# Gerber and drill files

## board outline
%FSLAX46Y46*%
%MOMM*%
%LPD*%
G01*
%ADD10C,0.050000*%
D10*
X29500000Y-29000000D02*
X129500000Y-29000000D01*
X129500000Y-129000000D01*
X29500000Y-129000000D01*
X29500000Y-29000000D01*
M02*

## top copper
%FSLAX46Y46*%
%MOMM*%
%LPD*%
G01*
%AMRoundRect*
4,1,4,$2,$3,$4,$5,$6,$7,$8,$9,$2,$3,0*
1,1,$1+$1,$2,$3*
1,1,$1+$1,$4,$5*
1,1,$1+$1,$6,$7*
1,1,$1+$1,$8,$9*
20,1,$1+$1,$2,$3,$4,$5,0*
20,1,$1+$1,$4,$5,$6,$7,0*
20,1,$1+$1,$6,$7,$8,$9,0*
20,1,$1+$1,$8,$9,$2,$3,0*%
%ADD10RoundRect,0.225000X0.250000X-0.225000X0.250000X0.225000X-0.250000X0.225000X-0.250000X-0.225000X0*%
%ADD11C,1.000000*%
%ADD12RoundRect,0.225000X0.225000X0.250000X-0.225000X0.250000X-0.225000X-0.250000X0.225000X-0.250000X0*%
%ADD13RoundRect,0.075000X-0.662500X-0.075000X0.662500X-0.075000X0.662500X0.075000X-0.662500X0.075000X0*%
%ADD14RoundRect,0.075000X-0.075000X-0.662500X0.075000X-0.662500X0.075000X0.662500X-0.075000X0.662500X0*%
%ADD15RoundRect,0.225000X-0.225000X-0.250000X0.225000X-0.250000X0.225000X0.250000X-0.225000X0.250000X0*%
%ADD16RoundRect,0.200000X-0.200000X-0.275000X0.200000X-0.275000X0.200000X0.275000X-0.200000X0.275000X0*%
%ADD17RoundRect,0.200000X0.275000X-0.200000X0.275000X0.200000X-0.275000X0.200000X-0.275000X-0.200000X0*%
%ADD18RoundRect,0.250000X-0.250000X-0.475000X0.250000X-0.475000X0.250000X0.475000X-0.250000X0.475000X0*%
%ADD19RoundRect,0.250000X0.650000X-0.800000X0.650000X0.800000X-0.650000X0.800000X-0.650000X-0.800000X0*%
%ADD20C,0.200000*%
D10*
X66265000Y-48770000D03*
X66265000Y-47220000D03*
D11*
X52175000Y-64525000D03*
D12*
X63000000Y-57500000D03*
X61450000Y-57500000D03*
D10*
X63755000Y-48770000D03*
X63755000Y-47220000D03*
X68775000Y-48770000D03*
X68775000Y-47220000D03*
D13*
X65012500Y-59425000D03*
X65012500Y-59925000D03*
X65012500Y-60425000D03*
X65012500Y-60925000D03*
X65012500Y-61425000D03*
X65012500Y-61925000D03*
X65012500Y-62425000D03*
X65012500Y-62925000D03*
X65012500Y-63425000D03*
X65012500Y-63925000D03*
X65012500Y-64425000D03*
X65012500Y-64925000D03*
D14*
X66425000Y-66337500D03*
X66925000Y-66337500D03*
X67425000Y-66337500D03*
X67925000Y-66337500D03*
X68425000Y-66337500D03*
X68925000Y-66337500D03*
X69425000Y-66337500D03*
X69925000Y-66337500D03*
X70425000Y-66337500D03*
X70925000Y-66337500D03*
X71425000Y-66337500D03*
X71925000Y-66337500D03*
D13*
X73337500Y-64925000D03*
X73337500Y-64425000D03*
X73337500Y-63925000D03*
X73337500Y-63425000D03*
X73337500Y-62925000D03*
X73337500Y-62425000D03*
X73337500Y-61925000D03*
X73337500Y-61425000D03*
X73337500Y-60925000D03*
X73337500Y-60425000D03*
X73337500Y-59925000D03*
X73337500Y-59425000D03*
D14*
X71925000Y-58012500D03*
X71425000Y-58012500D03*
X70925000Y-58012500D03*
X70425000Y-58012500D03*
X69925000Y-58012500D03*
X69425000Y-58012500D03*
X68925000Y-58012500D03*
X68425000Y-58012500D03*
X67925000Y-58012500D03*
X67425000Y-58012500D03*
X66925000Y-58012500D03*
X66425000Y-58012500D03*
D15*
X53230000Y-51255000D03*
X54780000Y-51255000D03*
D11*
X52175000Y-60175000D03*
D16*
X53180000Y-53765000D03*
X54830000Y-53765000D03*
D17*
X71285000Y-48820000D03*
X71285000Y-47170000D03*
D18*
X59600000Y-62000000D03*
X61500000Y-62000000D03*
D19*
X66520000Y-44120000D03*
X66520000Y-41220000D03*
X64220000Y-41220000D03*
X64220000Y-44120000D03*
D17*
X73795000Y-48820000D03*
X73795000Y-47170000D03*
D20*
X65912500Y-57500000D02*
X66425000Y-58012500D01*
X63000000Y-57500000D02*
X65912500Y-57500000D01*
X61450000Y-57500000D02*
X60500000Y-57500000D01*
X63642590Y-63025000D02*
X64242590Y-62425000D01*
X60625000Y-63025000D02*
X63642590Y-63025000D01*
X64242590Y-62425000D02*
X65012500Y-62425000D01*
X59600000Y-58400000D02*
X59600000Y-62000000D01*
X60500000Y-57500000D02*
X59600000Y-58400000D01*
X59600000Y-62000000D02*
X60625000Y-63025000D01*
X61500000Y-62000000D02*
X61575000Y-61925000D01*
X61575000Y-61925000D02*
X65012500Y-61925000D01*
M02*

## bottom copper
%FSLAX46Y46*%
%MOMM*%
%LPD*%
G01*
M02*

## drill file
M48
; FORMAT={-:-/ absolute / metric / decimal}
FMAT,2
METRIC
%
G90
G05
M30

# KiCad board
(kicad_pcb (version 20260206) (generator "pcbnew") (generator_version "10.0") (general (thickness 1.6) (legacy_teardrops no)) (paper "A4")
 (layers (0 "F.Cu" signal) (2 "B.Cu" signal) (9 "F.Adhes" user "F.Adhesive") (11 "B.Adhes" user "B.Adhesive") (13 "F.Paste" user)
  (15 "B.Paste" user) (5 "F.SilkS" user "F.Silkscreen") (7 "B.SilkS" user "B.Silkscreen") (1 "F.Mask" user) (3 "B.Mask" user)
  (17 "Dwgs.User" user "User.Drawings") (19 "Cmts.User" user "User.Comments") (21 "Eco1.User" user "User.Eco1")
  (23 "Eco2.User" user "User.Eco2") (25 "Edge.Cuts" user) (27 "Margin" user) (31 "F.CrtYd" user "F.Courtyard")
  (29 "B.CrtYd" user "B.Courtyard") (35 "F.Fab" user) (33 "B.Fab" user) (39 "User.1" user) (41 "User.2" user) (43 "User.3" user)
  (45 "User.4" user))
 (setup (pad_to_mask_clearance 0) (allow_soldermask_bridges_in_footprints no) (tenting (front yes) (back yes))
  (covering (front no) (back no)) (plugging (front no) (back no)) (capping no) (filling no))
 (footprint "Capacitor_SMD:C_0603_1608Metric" (layer "F.Cu") (at 66.265 47.995 90)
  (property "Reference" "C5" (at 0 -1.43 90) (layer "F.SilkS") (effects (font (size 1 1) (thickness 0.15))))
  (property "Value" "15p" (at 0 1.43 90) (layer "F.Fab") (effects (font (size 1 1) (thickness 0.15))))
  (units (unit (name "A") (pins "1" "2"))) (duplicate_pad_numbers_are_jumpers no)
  (pad "1" smd roundrect (at -0.775 0 90) (size 0.9 0.95) (layers "F.Cu" "F.Mask" "F.Paste") (roundrect_rratio 0.25) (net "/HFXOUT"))
  (pad "2" smd roundrect (at 0.775 0 90) (size 0.9 0.95) (layers "F.Cu" "F.Mask" "F.Paste") (roundrect_rratio 0.25) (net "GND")))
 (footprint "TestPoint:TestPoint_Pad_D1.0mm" (layer "F.Cu") (at 52.175 64.525)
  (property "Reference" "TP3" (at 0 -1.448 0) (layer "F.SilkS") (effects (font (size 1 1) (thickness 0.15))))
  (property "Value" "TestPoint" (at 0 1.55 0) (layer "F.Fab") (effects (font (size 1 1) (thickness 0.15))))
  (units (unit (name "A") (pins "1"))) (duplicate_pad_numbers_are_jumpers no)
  (pad "1" smd circle (at 0 0) (size 1 1) (layers "F.Cu" "F.Mask") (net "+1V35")))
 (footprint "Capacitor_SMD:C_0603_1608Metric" (layer "F.Cu") (at 62.225 57.5 180)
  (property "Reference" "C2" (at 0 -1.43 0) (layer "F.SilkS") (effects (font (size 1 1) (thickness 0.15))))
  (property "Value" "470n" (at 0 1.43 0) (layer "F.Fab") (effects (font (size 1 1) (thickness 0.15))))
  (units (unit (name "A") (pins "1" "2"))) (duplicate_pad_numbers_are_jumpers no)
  (pad "1" smd roundrect (at -0.775 0 180) (size 0.9 0.95) (layers "F.Cu" "F.Mask" "F.Paste") (roundrect_rratio 0.25) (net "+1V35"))
  (pad "2" smd roundrect (at 0.775 0 180) (size 0.9 0.95) (layers "F.Cu" "F.Mask" "F.Paste") (roundrect_rratio 0.25) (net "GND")))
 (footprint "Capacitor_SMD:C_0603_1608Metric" (layer "F.Cu") (at 63.755 47.995 90)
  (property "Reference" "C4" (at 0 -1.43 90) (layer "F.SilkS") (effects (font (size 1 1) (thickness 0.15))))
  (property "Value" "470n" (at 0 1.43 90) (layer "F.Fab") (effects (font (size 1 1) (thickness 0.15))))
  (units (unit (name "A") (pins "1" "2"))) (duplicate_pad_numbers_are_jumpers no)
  (pad "1" smd roundrect (at -0.775 0 90) (size 0.9 0.95) (layers "F.Cu" "F.Mask" "F.Paste") (roundrect_rratio 0.25) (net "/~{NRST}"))
  (pad "2" smd roundrect (at 0.775 0 90) (size 0.9 0.95) (layers "F.Cu" "F.Mask" "F.Paste") (roundrect_rratio 0.25) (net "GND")))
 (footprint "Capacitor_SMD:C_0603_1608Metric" (layer "F.Cu") (at 68.775 47.995 90)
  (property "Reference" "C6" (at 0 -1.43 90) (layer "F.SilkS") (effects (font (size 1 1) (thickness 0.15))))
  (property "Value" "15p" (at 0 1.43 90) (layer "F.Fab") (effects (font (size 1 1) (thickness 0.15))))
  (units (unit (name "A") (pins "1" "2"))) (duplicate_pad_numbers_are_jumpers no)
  (pad "1" smd roundrect (at -0.775 0 90) (size 0.9 0.95) (layers "F.Cu" "F.Mask" "F.Paste") (roundrect_rratio 0.25) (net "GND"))
  (pad "2" smd roundrect (at 0.775 0 90) (size 0.9 0.95) (layers "F.Cu" "F.Mask" "F.Paste") (roundrect_rratio 0.25) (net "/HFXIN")))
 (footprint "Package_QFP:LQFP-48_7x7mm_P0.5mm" (layer "F.Cu") (at 69.175 62.175)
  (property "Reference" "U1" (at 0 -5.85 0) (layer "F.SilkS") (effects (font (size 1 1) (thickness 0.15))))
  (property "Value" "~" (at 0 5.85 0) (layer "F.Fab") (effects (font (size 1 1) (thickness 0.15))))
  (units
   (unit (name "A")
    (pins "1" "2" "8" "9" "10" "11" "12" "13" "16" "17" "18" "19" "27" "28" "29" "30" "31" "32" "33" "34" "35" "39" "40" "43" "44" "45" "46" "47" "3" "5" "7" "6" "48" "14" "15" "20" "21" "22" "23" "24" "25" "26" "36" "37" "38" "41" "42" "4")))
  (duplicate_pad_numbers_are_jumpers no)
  (pad "1" smd roundrect (at -4.1625 -2.75) (size 1.475 0.3) (layers "F.Cu" "F.Mask" "F.Paste") (roundrect_rratio 0.25)
   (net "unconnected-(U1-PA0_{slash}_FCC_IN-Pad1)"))
  (pad "2" smd roundrect (at -4.1625 -2.25) (size 1.475 0.3) (layers "F.Cu" "F.Mask" "F.Paste") (roundrect_rratio 0.25)
   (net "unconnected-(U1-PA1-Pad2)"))
  (pad "3" smd roundrect (at -4.1625 -1.75) (size 1.475 0.3) (layers "F.Cu" "F.Mask" "F.Paste") (roundrect_rratio 0.25)
   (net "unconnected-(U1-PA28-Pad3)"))
  (pad "4" smd roundrect (at -4.1625 -1.25) (size 1.475 0.3) (layers "F.Cu" "F.Mask" "F.Paste") (roundrect_rratio 0.25) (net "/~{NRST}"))
  (pad "5" smd roundrect (at -4.1625 -0.75) (size 1.475 0.3) (layers "F.Cu" "F.Mask" "F.Paste") (roundrect_rratio 0.25)
   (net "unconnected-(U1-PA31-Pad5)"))
  (pad "6" smd roundrect (at -4.1625 -0.25) (size 1.475 0.3) (layers "F.Cu" "F.Mask" "F.Paste") (roundrect_rratio 0.25) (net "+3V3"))
  (pad "7" smd roundrect (at -4.1625 0.25) (size 1.475 0.3) (layers "F.Cu" "F.Mask" "F.Paste") (roundrect_rratio 0.25) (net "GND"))
  (pad "8" smd roundrect (at -4.1625 0.75) (size 1.475 0.3) (layers "F.Cu" "F.Mask" "F.Paste") (roundrect_rratio 0.25) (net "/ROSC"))
  (pad "9" smd roundrect (at -4.1625 1.25) (size 1.475 0.3) (layers "F.Cu" "F.Mask" "F.Paste") (roundrect_rratio 0.25)
   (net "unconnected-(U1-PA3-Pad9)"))
  (pad "10" smd roundrect (at -4.1625 1.75) (size 1.475 0.3) (layers "F.Cu" "F.Mask" "F.Paste") (roundrect_rratio 0.25)
   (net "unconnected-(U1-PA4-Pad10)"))
  (pad "11" smd roundrect (at -4.1625 2.25) (size 1.475 0.3) (layers "F.Cu" "F.Mask" "F.Paste") (roundrect_rratio 0.25) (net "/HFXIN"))
  (pad "12" smd roundrect (at -4.1625 2.75) (size 1.475 0.3) (layers "F.Cu" "F.Mask" "F.Paste") (roundrect_rratio 0.25) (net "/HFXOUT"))
  (pad "13" smd roundrect (at -2.75 4.1625) (size 0.3 1.475) (layers "F.Cu" "F.Mask" "F.Paste") (roundrect_rratio 0.25)
   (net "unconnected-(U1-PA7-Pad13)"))
  (pad "14" smd roundrect (at -2.25 4.1625) (size 0.3 1.475) (layers "F.Cu" "F.Mask" "F.Paste") (roundrect_rratio 0.25)
   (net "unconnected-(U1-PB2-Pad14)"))
  (pad "15" smd roundrect (at -1.75 4.1625) (size 0.3 1.475) (layers "F.Cu" "F.Mask" "F.Paste") (roundrect_rratio 0.25)
   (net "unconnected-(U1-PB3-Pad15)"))
  (pad "16" smd roundrect (at -1.25 4.1625) (size 0.3 1.475) (layers "F.Cu" "F.Mask" "F.Paste") (roundrect_rratio 0.25)
   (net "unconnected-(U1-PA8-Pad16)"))
  (pad "17" smd roundrect (at -0.75 4.1625) (size 0.3 1.475) (layers "F.Cu" "F.Mask" "F.Paste") (roundrect_rratio 0.25)
   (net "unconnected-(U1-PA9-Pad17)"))
  (pad "18" smd roundrect (at -0.25 4.1625) (size 0.3 1.475) (layers "F.Cu" "F.Mask" "F.Paste") (roundrect_rratio 0.25)
   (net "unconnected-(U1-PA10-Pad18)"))
  (pad "19" smd roundrect (at 0.25 4.1625) (size 0.3 1.475) (layers "F.Cu" "F.Mask" "F.Paste") (roundrect_rratio 0.25)
   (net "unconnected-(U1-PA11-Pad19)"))
  (pad "20" smd roundrect (at 0.75 4.1625) (size 0.3 1.475) (layers "F.Cu" "F.Mask" "F.Paste") (roundrect_rratio 0.25)
   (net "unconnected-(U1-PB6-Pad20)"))
  (pad "21" smd roundrect (at 1.25 4.1625) (size 0.3 1.475) (layers "F.Cu" "F.Mask" "F.Paste") (roundrect_rratio 0.25)
   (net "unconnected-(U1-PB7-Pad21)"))
  (pad "22" smd roundrect (at 1.75 4.1625) (size 0.3 1.475) (layers "F.Cu" "F.Mask" "F.Paste") (roundrect_rratio 0.25)
   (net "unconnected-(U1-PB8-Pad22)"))
  (pad "23" smd roundrect (at 2.25 4.1625) (size 0.3 1.475) (layers "F.Cu" "F.Mask" "F.Paste") (roundrect_rratio 0.25)
   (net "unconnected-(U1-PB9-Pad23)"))
  (pad "24" smd roundrect (at 2.75 4.1625) (size 0.3 1.475) (layers "F.Cu" "F.Mask" "F.Paste") (roundrect_rratio 0.25)
   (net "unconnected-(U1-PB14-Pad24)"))
  (pad "25" smd roundrect (at 4.1625 2.75) (size 1.475 0.3) (layers "F.Cu" "F.Mask" "F.Paste") (roundrect_rratio 0.25)
   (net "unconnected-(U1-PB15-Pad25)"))
  (pad "26" smd roundrect (at 4.1625 2.25) (size 1.475 0.3) (layers "F.Cu" "F.Mask" "F.Paste") (roundrect_rratio 0.25)
   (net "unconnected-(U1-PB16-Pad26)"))
  (pad "27" smd roundrect (at 4.1625 1.75) (size 1.475 0.3) (layers "F.Cu" "F.Mask" "F.Paste") (roundrect_rratio 0.25)
   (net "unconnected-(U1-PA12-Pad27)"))
  (pad "28" smd roundrect (at 4.1625 1.25) (size 1.475 0.3) (layers "F.Cu" "F.Mask" "F.Paste") (roundrect_rratio 0.25)
   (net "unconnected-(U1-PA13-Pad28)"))
  (pad "29" smd roundrect (at 4.1625 0.75) (size 1.475 0.3) (layers "F.Cu" "F.Mask" "F.Paste") (roundrect_rratio 0.25)
   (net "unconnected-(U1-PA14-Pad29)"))
  (pad "30" smd roundrect (at 4.1625 0.25) (size 1.475 0.3) (layers "F.Cu" "F.Mask" "F.Paste") (roundrect_rratio 0.25)
   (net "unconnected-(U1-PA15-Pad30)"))
  (pad "31" smd roundrect (at 4.1625 -0.25) (size 1.475 0.3) (layers "F.Cu" "F.Mask" "F.Paste") (roundrect_rratio 0.25)
   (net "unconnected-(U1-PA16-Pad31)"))
  (pad "32" smd roundrect (at 4.1625 -0.75) (size 1.475 0.3) (layers "F.Cu" "F.Mask" "F.Paste") (roundrect_rratio 0.25)
   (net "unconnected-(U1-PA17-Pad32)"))
  (pad "33" smd roundrect (at 4.1625 -1.25) (size 1.475 0.3) (layers "F.Cu" "F.Mask" "F.Paste") (roundrect_rratio 0.25)
   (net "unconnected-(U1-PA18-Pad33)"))
  (pad "34" smd roundrect (at 4.1625 -1.75) (size 1.475 0.3) (layers "F.Cu" "F.Mask" "F.Paste") (roundrect_rratio 0.25)
   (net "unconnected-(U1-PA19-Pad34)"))
  (pad "35" smd roundrect (at 4.1625 -2.25) (size 1.475 0.3) (layers "F.Cu" "F.Mask" "F.Paste") (roundrect_rratio 0.25)
   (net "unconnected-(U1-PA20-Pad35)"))
  (pad "36" smd roundrect (at 4.1625 -2.75) (size 1.475 0.3) (layers "F.Cu" "F.Mask" "F.Paste") (roundrect_rratio 0.25)
   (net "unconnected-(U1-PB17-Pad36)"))
  (pad "37" smd roundrect (at 2.75 -4.1625) (size 0.3 1.475) (layers "F.Cu" "F.Mask" "F.Paste") (roundrect_rratio 0.25)
   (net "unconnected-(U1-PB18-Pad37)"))
  (pad "38" smd roundrect (at 2.25 -4.1625) (size 0.3 1.475) (layers "F.Cu" "F.Mask" "F.Paste") (roundrect_rratio 0.25)
   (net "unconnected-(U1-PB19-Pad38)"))
  (pad "39" smd roundrect (at 1.75 -4.1625) (size 0.3 1.475) (layers "F.Cu" "F.Mask" "F.Paste") (roundrect_rratio 0.25) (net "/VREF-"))
  (pad "40" smd roundrect (at 1.25 -4.1625) (size 0.3 1.475) (layers "F.Cu" "F.Mask" "F.Paste") (roundrect_rratio 0.25)
   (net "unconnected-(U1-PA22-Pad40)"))
  (pad "41" smd roundrect (at 0.75 -4.1625) (size 0.3 1.475) (layers "F.Cu" "F.Mask" "F.Paste") (roundrect_rratio 0.25)
   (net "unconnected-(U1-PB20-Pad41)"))
  (pad "42" smd roundrect (at 0.25 -4.1625) (size 0.3 1.475) (layers "F.Cu" "F.Mask" "F.Paste") (roundrect_rratio 0.25)
   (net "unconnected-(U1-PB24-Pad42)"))
  (pad "43" smd roundrect (at -0.25 -4.1625) (size 0.3 1.475) (layers "F.Cu" "F.Mask" "F.Paste") (roundrect_rratio 0.25) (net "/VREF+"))
  (pad "44" smd roundrect (at -0.75 -4.1625) (size 0.3 1.475) (layers "F.Cu" "F.Mask" "F.Paste") (roundrect_rratio 0.25)
   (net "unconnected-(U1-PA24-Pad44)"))
  (pad "45" smd roundrect (at -1.25 -4.1625) (size 0.3 1.475) (layers "F.Cu" "F.Mask" "F.Paste") (roundrect_rratio 0.25)
   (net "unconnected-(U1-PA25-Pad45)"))
  (pad "46" smd roundrect (at -1.75 -4.1625) (size 0.3 1.475) (layers "F.Cu" "F.Mask" "F.Paste") (roundrect_rratio 0.25)
   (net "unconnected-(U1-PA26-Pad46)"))
  (pad "47" smd roundrect (at -2.25 -4.1625) (size 0.3 1.475) (layers "F.Cu" "F.Mask" "F.Paste") (roundrect_rratio 0.25)
   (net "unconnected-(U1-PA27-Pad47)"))
  (pad "48" smd roundrect (at -2.75 -4.1625) (size 0.3 1.475) (layers "F.Cu" "F.Mask" "F.Paste") (roundrect_rratio 0.25) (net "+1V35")))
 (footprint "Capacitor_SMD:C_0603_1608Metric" (layer "F.Cu") (at 54.005 51.255)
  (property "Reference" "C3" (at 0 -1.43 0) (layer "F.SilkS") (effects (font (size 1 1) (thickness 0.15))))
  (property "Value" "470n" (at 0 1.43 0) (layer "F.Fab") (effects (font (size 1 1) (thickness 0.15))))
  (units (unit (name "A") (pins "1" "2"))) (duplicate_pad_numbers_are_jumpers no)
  (pad "1" smd roundrect (at -0.775 0) (size 0.9 0.95) (layers "F.Cu" "F.Mask" "F.Paste") (roundrect_rratio 0.25) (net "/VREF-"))
  (pad "2" smd roundrect (at 0.775 0) (size 0.9 0.95) (layers "F.Cu" "F.Mask" "F.Paste") (roundrect_rratio 0.25) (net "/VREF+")))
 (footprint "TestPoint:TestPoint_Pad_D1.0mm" (layer "F.Cu") (at 52.175 60.175)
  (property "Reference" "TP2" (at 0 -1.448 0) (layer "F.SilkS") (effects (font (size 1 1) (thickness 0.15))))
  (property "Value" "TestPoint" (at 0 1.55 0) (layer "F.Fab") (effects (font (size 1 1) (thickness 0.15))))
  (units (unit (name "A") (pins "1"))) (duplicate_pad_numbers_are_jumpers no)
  (pad "1" smd circle (at 0 0) (size 1 1) (layers "F.Cu" "F.Mask") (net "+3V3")))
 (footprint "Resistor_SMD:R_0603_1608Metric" (layer "F.Cu") (at 54.005 53.765)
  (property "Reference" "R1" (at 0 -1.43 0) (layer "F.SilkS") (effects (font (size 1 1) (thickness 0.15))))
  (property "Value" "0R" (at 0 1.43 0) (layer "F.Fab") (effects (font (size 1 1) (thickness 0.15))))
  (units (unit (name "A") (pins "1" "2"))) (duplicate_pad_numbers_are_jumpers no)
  (pad "1" smd roundrect (at -0.825 0) (size 0.8 0.95) (layers "F.Cu" "F.Mask" "F.Paste") (roundrect_rratio 0.25) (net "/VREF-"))
  (pad "2" smd roundrect (at 0.825 0) (size 0.8 0.95) (layers "F.Cu" "F.Mask" "F.Paste") (roundrect_rratio 0.25) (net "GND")))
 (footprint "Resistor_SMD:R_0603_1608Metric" (layer "F.Cu") (at 71.285 47.995 90)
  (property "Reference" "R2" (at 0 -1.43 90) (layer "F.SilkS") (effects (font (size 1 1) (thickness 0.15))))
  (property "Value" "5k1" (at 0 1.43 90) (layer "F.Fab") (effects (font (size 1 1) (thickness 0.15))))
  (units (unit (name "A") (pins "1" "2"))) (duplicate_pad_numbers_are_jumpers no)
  (pad "1" smd roundrect (at -0.825 0 90) (size 0.8 0.95) (layers "F.Cu" "F.Mask" "F.Paste") (roundrect_rratio 0.25) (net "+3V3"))
  (pad "2" smd roundrect (at 0.825 0 90) (size 0.8 0.95) (layers "F.Cu" "F.Mask" "F.Paste") (roundrect_rratio 0.25) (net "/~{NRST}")))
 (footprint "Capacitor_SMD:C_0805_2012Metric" (layer "F.Cu") (at 60.55 62)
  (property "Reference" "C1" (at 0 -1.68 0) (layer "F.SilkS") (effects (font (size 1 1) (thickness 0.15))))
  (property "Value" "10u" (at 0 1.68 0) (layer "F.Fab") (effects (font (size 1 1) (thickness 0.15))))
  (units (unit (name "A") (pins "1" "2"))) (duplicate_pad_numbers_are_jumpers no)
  (pad "1" smd roundrect (at -0.95 0) (size 1 1.45) (layers "F.Cu" "F.Mask" "F.Paste") (roundrect_rratio 0.25) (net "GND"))
  (pad "2" smd roundrect (at 0.95 0) (size 1 1.45) (layers "F.Cu" "F.Mask" "F.Paste") (roundrect_rratio 0.25) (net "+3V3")))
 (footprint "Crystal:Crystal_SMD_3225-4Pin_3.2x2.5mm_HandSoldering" (layer "F.Cu") (at 65.37 42.67 90)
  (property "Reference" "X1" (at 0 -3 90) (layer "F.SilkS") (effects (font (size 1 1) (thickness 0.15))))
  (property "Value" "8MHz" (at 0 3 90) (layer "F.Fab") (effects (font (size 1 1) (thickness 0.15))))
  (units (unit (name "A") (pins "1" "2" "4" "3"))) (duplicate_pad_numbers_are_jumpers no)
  (pad "1" smd roundrect (at -1.45 1.15 90) (size 2.1 1.8) (layers "F.Cu" "F.Mask" "F.Paste") (roundrect_rratio 0.138889) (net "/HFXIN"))
  (pad "2" smd roundrect (at 1.45 1.15 90) (size 2.1 1.8) (layers "F.Cu" "F.Mask" "F.Paste") (roundrect_rratio 0.138889) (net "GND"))
  (pad "3" smd roundrect (at 1.45 -1.15 90) (size 2.1 1.8) (layers "F.Cu" "F.Mask" "F.Paste") (roundrect_rratio 0.138889) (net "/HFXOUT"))
  (pad "4" smd roundrect (at -1.45 -1.15 90) (size 2.1 1.8) (layers "F.Cu" "F.Mask" "F.Paste") (roundrect_rratio 0.138889) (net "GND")))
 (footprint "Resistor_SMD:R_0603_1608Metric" (layer "F.Cu") (at 73.795 47.995 90)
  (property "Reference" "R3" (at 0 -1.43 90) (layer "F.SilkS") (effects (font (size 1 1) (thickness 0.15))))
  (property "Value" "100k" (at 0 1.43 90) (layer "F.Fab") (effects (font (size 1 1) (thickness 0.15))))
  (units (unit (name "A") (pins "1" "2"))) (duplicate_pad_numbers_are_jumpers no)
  (pad "1" smd roundrect (at -0.825 0 90) (size 0.8 0.95) (layers "F.Cu" "F.Mask" "F.Paste") (roundrect_rratio 0.25) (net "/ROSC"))
  (pad "2" smd roundrect (at 0.825 0 90) (size 0.8 0.95) (layers "F.Cu" "F.Mask" "F.Paste") (roundrect_rratio 0.25) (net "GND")))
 (gr_rect (start 29.5 29) (end 129.5 129) (stroke (width 0.05) (type solid)) (fill no) (layer "Edge.Cuts"))
 (segment (start 65.9125 57.5) (end 66.425 58.0125) (width 0.2) (layer "F.Cu") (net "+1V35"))
 (segment (start 63 57.5) (end 65.9125 57.5) (width 0.2) (layer "F.Cu") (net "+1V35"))
 (segment (start 61.45 57.5) (end 60.5 57.5) (width 0.2) (layer "F.Cu") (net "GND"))
 (segment (start 63.64259 63.025) (end 64.24259 62.425) (width 0.2) (layer "F.Cu") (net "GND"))
 (segment (start 60.625 63.025) (end 63.64259 63.025) (width 0.2) (layer "F.Cu") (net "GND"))
 (segment (start 64.24259 62.425) (end 65.0125 62.425) (width 0.2) (layer "F.Cu") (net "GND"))
 (segment (start 59.6 58.4) (end 59.6 62) (width 0.2) (layer "F.Cu") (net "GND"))
 (segment (start 60.5 57.5) (end 59.6 58.4) (width 0.2) (layer "F.Cu") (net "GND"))
 (segment (start 59.6 62) (end 60.625 63.025) (width 0.2) (layer "F.Cu") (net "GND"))
 (segment (start 61.5 62) (end 61.575 61.925) (width 0.2) (layer "F.Cu") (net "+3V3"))
 (segment (start 61.575 61.925) (end 65.0125 61.925) (width 0.2) (layer "F.Cu") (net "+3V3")))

